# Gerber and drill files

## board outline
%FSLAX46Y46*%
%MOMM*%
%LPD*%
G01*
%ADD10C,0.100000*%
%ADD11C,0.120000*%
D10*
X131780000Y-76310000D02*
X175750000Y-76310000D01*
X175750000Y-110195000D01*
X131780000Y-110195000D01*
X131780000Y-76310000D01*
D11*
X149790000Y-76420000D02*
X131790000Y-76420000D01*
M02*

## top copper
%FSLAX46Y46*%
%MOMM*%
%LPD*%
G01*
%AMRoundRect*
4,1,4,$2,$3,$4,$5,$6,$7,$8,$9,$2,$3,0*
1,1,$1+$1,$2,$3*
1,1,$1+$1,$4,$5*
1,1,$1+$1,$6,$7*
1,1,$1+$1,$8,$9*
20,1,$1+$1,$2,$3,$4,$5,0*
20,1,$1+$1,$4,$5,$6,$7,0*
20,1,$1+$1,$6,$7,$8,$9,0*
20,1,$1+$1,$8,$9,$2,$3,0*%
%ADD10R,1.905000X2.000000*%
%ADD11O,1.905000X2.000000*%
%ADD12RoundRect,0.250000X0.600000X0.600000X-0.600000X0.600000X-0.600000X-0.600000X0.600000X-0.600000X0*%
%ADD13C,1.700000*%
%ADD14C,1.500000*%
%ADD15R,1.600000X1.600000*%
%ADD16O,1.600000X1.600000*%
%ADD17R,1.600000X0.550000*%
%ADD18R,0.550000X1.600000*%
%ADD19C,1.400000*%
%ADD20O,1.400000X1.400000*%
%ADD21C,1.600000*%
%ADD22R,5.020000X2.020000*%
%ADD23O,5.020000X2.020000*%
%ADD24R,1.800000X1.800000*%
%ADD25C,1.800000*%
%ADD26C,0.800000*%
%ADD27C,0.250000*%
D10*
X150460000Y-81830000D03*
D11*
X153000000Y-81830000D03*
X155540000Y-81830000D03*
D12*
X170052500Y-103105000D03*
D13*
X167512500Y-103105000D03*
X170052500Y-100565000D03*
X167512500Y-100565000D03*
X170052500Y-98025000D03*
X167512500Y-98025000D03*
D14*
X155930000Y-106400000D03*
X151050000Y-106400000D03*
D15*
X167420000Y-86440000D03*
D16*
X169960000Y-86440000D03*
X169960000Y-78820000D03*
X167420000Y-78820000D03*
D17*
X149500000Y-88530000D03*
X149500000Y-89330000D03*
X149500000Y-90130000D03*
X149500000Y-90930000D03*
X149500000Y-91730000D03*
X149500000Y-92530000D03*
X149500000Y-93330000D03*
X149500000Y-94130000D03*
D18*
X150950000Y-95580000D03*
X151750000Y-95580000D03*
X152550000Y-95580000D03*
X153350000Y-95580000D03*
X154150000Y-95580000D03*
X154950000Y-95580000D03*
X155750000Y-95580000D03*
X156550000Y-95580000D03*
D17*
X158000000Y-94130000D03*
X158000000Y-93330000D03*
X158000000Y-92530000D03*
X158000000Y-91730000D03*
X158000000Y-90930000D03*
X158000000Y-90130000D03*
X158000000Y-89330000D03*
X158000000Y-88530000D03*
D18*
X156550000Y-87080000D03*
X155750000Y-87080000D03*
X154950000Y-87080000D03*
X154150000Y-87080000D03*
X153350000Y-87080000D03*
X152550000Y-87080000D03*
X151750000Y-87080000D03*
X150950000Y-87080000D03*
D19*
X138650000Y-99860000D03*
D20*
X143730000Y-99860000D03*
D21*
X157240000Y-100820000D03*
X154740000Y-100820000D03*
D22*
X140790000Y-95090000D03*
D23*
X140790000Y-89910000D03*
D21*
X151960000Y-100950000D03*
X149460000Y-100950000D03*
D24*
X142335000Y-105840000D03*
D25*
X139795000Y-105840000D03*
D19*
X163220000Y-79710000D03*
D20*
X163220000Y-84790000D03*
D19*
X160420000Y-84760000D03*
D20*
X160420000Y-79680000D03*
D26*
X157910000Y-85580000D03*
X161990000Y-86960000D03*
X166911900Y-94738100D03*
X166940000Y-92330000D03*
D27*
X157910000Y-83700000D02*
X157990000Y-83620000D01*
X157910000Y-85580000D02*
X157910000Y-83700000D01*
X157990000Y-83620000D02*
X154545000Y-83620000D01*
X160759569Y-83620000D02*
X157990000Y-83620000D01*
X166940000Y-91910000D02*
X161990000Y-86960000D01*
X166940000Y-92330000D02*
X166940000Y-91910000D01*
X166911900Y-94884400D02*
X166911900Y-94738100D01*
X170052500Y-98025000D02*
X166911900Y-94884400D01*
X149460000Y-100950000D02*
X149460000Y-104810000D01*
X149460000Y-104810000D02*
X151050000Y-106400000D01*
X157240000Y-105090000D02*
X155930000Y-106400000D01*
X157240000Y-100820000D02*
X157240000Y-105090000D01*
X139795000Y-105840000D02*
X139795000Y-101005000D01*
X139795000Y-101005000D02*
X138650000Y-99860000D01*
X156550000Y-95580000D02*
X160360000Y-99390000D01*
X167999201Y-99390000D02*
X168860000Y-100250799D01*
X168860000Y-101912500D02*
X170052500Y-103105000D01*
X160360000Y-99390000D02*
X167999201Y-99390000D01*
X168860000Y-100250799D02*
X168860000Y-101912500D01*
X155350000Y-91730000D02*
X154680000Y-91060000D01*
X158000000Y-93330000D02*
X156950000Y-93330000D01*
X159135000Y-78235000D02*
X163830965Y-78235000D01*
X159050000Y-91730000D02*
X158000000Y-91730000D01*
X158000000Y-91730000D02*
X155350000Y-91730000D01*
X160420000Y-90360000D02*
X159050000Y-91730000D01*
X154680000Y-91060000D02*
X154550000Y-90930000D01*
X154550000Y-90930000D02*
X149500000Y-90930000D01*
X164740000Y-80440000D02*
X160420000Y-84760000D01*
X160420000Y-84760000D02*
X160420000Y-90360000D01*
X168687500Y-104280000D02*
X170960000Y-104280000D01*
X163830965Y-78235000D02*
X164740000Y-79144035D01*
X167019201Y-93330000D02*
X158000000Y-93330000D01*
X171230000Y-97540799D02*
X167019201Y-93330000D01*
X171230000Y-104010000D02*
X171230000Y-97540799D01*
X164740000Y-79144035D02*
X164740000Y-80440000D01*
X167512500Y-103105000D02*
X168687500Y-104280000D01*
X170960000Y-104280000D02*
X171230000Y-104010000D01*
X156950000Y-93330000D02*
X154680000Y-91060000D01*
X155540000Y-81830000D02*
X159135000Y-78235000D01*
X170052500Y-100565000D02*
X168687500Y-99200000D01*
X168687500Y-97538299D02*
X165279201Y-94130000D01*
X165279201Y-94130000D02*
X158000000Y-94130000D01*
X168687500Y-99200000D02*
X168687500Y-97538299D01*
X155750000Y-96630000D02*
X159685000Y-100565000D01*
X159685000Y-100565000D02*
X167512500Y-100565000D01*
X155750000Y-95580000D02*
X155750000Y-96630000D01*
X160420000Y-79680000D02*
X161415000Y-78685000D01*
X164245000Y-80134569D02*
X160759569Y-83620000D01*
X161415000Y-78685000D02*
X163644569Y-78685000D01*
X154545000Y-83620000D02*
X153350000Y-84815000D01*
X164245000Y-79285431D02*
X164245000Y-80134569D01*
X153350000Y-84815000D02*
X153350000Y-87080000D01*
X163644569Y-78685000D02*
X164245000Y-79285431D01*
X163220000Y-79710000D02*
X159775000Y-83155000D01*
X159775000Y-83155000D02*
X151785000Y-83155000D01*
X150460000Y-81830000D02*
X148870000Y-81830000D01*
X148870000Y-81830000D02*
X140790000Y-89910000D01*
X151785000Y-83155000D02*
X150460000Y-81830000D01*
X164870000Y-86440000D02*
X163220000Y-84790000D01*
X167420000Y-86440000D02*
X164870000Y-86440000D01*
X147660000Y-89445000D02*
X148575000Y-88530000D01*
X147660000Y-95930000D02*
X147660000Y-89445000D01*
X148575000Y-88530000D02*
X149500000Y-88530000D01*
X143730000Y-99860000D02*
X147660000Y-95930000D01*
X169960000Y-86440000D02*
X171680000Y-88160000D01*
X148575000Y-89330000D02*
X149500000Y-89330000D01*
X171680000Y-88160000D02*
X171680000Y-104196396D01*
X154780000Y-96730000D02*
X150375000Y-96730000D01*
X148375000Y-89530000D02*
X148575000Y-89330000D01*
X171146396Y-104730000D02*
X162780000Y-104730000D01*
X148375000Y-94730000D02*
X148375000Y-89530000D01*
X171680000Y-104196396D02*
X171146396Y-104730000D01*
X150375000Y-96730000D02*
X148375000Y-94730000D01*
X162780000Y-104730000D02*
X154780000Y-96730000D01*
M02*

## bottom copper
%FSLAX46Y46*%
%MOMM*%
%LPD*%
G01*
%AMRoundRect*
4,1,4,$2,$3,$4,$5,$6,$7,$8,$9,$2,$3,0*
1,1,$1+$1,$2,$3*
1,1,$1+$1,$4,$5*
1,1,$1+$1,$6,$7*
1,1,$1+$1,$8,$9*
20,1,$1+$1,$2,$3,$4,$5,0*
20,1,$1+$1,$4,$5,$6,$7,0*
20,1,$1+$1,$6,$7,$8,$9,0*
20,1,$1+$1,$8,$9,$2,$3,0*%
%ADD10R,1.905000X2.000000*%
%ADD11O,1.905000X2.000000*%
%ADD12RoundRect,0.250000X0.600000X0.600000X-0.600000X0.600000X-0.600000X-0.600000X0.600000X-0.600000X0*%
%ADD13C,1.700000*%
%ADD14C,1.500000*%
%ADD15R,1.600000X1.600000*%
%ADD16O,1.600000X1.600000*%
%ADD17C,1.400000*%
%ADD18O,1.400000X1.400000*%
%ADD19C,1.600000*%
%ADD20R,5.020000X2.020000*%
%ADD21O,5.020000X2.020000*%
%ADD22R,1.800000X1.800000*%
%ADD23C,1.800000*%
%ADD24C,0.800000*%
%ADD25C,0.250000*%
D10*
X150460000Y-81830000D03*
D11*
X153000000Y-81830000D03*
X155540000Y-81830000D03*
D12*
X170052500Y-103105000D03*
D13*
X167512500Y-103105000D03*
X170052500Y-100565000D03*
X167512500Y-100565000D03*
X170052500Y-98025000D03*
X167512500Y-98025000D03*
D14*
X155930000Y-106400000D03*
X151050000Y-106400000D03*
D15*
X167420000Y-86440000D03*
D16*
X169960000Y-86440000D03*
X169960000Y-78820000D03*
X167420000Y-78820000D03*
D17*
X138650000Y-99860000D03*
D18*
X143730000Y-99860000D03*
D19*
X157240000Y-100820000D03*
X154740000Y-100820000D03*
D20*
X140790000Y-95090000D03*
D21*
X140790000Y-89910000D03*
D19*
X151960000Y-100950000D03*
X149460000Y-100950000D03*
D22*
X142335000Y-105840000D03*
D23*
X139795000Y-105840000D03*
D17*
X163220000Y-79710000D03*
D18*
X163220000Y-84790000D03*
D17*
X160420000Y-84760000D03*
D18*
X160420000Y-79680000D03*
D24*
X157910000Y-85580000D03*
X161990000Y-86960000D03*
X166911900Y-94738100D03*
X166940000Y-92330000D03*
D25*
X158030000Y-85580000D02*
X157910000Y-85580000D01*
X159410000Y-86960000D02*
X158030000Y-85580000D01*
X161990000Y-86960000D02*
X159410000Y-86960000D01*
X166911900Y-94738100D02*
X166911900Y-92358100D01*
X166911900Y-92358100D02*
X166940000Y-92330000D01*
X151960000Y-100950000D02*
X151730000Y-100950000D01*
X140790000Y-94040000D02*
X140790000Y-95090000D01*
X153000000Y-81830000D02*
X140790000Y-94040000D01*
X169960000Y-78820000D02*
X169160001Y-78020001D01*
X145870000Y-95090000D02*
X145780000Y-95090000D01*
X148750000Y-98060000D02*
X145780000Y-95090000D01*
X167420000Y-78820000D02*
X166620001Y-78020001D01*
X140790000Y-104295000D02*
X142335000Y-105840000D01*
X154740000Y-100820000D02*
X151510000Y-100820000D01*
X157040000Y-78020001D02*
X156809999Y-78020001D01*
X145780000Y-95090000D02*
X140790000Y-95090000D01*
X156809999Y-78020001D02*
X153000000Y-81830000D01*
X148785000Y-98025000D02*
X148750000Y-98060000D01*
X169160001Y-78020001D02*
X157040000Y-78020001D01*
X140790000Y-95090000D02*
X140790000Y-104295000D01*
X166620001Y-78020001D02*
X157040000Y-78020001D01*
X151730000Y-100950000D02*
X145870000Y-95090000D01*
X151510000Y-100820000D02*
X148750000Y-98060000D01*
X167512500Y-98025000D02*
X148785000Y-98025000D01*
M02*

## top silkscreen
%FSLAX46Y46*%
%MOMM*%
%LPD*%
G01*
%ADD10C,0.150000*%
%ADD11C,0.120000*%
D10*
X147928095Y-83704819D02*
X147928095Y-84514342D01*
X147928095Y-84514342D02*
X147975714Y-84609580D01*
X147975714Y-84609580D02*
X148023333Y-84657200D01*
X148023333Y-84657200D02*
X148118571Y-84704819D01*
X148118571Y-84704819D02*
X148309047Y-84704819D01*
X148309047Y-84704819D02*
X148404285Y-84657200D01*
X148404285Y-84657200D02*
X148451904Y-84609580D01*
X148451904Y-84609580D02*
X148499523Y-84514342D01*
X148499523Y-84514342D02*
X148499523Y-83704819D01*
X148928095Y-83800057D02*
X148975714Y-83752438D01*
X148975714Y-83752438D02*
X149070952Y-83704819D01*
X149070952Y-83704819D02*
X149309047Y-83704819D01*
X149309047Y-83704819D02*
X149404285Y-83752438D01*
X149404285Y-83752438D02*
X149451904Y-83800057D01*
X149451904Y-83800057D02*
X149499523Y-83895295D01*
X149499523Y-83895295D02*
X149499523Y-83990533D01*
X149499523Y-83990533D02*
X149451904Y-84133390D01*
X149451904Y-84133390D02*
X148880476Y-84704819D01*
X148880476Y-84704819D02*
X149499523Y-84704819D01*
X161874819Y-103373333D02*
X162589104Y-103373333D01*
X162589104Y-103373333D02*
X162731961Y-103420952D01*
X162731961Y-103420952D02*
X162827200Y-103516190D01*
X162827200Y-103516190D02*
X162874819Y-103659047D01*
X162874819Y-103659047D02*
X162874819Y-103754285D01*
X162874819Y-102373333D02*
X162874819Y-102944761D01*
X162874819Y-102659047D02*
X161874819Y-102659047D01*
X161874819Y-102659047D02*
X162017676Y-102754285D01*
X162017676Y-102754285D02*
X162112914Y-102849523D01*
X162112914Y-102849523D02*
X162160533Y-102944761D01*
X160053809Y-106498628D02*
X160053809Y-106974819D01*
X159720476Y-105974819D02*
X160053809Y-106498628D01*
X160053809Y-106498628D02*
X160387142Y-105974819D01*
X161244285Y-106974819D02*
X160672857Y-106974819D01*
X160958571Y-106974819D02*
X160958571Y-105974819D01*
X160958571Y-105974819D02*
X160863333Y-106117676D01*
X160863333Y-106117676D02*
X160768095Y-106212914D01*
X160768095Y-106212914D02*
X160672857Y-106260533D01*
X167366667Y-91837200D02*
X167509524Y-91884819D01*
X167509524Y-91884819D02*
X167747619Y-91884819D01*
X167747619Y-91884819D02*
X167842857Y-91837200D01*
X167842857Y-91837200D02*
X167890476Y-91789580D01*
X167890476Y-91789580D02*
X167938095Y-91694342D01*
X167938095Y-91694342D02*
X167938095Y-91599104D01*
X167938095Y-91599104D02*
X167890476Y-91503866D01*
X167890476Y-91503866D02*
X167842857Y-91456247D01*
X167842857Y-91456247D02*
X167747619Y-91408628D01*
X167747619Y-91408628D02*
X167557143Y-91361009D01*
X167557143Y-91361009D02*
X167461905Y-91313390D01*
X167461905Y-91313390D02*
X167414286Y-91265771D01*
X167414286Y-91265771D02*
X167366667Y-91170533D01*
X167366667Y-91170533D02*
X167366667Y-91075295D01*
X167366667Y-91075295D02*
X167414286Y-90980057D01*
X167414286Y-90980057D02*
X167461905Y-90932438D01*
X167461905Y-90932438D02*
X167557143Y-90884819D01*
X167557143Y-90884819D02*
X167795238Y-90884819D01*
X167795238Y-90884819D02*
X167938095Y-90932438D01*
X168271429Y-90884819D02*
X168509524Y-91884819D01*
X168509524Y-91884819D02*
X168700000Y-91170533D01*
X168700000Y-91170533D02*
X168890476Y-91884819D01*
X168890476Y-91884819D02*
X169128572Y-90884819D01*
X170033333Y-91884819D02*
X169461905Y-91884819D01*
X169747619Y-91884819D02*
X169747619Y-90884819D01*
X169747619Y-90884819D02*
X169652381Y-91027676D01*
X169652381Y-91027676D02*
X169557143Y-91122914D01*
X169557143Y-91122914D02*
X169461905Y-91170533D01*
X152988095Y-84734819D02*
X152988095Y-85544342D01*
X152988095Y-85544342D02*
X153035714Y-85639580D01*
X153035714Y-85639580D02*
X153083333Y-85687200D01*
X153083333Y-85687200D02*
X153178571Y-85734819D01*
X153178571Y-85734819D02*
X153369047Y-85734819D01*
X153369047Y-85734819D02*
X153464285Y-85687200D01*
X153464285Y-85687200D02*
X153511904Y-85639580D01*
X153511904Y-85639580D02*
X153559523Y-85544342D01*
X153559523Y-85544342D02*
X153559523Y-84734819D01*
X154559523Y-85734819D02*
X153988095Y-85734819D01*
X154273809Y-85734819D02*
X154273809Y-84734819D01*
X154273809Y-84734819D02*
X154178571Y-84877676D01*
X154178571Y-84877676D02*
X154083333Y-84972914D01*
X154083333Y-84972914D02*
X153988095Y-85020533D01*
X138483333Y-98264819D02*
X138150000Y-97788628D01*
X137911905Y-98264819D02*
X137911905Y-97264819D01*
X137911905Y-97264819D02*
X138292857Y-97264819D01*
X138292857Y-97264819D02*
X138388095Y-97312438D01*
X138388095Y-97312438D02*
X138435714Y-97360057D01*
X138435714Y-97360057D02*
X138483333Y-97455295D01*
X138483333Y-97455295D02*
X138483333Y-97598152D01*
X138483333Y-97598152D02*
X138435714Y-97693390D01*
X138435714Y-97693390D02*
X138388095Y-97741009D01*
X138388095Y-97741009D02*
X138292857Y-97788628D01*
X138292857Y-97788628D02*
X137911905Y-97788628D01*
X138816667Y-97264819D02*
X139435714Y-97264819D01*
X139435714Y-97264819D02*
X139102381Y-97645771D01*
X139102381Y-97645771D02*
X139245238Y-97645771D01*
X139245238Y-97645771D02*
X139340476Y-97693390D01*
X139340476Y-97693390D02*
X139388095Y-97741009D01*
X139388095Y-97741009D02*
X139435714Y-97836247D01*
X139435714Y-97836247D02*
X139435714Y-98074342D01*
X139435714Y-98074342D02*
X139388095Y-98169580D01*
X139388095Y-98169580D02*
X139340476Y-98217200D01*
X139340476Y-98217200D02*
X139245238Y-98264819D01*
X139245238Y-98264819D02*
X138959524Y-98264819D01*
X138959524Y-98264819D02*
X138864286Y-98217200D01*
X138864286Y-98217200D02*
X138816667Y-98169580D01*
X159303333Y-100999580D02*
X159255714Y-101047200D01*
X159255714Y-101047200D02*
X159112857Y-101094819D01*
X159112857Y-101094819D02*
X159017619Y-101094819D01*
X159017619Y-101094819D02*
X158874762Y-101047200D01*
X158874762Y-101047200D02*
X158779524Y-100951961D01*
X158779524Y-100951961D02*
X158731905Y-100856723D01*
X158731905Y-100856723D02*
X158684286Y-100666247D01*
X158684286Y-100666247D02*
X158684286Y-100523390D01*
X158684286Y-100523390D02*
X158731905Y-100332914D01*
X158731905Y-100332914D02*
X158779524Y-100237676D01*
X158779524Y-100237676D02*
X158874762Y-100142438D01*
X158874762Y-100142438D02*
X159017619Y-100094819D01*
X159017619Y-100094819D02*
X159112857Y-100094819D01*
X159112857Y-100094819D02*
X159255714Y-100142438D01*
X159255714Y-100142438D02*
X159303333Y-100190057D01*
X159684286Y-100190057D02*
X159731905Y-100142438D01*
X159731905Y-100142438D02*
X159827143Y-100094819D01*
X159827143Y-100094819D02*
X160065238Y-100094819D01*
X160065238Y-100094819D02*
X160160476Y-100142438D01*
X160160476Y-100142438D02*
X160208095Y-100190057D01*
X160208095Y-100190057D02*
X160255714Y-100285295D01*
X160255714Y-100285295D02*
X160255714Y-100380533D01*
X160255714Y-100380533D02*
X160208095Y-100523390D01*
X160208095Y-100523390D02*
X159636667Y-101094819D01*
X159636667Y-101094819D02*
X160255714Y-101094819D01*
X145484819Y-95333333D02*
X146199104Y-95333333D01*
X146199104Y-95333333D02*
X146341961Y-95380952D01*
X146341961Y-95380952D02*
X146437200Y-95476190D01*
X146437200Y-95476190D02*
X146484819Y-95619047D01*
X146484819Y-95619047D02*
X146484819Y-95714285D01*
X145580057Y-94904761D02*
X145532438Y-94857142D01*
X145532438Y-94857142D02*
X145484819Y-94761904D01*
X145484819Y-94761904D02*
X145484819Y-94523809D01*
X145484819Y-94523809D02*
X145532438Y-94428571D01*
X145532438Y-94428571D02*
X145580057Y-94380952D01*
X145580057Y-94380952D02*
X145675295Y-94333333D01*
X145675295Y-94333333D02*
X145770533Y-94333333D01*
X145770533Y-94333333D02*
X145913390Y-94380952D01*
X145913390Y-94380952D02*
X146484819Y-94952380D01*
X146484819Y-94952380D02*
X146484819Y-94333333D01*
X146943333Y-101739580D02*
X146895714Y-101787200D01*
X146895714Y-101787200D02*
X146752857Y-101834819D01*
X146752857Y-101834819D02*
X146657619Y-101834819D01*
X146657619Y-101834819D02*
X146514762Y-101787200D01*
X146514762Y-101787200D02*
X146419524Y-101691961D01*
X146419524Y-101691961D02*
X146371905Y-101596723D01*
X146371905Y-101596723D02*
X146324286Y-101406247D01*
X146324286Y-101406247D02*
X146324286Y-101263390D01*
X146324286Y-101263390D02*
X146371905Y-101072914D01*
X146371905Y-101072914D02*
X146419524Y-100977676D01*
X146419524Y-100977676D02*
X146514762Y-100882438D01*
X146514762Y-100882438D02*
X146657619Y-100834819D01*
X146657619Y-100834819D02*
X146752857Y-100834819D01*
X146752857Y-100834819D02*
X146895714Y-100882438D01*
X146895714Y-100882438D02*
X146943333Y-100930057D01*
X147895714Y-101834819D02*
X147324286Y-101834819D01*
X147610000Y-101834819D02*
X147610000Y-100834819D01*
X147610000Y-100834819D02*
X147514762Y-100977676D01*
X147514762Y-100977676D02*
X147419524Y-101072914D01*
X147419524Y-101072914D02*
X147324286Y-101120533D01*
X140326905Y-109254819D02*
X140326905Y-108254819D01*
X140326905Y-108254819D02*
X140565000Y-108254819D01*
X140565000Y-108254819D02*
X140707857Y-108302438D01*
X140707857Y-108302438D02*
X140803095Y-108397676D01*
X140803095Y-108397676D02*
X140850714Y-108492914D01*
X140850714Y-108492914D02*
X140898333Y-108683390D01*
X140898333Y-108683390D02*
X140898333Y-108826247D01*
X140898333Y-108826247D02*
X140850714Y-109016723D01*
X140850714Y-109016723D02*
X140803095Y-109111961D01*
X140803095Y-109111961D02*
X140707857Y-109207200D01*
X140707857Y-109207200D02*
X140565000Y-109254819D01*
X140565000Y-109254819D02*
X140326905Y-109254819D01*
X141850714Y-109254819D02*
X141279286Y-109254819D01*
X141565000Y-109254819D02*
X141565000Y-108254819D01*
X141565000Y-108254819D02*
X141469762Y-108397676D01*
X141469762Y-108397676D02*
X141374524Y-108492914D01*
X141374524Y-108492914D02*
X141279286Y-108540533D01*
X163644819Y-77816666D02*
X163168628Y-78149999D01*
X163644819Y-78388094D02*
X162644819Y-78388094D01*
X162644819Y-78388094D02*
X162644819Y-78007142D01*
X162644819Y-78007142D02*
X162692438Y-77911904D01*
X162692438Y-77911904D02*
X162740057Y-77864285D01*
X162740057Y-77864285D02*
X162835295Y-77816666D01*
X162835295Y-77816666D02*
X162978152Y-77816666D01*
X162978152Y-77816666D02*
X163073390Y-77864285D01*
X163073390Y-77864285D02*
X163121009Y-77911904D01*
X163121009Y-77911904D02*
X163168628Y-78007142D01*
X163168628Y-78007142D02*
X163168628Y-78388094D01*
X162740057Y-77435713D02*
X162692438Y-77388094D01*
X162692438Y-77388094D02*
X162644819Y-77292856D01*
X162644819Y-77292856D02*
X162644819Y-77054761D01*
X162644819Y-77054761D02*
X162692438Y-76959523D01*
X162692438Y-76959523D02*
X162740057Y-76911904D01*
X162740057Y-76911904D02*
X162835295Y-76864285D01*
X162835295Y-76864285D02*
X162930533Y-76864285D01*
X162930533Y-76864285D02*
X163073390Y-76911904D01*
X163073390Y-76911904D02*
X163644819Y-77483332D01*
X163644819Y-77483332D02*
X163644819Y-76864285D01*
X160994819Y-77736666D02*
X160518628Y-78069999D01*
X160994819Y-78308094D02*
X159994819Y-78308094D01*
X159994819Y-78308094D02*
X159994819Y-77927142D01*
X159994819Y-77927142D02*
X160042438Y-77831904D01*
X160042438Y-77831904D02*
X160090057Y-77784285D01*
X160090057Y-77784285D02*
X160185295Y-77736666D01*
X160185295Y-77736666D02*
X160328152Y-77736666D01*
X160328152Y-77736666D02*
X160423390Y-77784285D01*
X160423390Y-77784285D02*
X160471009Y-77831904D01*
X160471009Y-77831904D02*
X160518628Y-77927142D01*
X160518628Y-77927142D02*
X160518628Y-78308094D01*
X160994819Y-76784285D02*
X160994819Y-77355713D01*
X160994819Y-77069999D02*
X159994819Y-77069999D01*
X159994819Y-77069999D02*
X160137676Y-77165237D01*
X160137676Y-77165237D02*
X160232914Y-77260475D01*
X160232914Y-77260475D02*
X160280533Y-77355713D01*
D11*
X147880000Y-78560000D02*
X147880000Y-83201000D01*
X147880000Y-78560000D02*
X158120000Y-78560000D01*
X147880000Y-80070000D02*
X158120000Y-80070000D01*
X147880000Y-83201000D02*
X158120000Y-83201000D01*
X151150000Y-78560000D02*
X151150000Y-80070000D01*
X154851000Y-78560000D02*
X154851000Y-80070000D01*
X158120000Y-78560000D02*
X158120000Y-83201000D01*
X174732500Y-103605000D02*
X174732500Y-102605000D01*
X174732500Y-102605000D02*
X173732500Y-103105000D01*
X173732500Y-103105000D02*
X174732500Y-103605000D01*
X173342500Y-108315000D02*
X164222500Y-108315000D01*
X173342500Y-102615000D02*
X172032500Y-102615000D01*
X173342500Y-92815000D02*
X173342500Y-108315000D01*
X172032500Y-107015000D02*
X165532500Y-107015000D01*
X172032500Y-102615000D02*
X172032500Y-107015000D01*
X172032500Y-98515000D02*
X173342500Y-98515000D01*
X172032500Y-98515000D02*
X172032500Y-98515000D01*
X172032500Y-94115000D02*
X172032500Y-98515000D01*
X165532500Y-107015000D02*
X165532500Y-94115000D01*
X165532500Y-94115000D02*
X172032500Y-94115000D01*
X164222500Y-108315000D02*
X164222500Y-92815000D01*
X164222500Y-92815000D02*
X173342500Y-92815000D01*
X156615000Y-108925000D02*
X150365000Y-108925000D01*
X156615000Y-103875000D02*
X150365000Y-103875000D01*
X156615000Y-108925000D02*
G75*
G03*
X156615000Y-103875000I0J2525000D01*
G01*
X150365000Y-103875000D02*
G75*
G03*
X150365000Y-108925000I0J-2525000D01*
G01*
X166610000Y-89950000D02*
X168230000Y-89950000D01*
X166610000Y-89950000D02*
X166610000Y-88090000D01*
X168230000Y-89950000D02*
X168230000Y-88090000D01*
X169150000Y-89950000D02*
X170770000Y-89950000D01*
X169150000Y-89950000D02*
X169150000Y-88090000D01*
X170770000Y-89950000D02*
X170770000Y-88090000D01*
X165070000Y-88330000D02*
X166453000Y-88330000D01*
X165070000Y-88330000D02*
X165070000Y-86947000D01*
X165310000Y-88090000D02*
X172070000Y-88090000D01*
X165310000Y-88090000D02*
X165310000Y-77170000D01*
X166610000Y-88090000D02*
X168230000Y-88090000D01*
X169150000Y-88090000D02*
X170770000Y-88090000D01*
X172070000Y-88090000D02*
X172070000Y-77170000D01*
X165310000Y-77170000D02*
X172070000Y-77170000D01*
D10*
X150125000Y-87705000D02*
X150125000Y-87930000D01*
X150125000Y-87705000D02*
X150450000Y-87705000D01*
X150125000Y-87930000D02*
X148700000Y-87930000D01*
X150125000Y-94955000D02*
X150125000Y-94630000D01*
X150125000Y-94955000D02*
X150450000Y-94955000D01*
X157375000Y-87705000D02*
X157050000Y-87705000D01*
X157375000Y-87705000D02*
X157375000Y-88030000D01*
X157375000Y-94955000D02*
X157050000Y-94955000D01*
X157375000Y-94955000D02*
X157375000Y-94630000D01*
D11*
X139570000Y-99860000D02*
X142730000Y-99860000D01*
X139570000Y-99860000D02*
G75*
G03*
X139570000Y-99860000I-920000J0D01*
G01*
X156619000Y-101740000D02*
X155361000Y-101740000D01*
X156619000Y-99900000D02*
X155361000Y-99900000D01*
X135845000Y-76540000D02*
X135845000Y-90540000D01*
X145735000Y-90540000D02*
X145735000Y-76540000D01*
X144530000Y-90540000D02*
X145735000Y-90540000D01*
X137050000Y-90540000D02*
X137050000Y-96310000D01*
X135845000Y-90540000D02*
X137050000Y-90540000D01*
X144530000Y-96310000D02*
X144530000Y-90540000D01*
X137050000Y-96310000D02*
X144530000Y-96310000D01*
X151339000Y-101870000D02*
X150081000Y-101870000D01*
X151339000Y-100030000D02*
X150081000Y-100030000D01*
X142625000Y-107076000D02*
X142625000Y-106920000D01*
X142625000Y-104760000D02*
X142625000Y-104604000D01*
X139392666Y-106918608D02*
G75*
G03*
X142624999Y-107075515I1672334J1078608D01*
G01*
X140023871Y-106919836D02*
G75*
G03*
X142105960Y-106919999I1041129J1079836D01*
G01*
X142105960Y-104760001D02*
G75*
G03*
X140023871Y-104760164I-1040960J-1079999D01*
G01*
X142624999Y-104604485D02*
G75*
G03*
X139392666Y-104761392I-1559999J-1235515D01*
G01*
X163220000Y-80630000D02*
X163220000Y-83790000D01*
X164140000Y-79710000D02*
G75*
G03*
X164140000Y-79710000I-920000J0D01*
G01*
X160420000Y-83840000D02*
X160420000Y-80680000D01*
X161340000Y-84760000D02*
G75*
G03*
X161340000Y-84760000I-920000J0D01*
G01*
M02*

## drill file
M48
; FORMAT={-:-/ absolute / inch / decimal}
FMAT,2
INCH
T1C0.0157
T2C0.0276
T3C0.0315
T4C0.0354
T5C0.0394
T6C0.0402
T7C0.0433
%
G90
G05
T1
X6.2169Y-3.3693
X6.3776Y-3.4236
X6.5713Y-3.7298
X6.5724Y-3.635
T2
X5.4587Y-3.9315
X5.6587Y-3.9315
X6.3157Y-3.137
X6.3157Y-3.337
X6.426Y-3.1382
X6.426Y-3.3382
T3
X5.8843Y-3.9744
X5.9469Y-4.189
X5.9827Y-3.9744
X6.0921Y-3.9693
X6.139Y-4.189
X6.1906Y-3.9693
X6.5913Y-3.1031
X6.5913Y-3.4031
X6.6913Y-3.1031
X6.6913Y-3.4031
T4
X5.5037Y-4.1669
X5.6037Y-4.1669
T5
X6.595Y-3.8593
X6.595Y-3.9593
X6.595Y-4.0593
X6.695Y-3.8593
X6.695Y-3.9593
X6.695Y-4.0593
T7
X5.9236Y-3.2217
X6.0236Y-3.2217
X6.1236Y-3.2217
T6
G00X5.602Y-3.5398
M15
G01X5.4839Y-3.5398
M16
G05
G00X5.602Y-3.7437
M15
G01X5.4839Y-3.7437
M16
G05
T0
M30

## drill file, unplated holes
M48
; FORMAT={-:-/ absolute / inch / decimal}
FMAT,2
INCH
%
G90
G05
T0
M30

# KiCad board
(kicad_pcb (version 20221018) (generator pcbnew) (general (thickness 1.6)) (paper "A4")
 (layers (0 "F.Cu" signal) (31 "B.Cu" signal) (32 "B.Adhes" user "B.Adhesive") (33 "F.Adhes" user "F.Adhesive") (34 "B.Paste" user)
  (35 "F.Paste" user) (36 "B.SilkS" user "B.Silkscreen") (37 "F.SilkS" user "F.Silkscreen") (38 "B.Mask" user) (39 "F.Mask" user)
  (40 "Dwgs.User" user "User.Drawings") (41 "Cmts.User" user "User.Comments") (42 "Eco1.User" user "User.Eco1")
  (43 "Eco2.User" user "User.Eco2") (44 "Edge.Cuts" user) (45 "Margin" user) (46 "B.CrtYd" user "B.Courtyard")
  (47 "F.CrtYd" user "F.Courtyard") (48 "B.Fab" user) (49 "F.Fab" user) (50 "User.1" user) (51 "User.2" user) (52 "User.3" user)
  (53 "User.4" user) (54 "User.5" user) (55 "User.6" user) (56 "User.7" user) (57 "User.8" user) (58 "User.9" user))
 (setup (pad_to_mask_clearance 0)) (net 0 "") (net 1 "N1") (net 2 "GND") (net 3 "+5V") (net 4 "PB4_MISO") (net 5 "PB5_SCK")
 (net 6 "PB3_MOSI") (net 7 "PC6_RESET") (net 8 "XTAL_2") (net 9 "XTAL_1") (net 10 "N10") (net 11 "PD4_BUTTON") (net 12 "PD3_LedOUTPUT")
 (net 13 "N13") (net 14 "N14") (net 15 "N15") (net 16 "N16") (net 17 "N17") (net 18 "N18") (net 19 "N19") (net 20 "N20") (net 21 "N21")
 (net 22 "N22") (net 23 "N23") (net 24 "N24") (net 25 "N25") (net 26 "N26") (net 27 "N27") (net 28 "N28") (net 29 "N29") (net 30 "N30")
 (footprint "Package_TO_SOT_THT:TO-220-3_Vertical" (layer "F.Cu") (at 150.46 81.83)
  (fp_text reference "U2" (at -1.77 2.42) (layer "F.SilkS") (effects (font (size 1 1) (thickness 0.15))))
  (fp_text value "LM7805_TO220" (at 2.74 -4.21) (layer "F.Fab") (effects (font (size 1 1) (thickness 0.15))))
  (fp_line (start -2.58 -3.27) (end -2.58 1.371) (stroke (width 0.12) (type solid)) (layer "F.SilkS"))
  (fp_line (start -2.58 -3.27) (end 7.66 -3.27) (stroke (width 0.12) (type solid)) (layer "F.SilkS"))
  (fp_line (start -2.58 -1.76) (end 7.66 -1.76) (stroke (width 0.12) (type solid)) (layer "F.SilkS"))
  (fp_line (start -2.58 1.371) (end 7.66 1.371) (stroke (width 0.12) (type solid)) (layer "F.SilkS"))
  (fp_line (start 0.69 -3.27) (end 0.69 -1.76) (stroke (width 0.12) (type solid)) (layer "F.SilkS"))
  (fp_line (start 4.391 -3.27) (end 4.391 -1.76) (stroke (width 0.12) (type solid)) (layer "F.SilkS"))
  (fp_line (start 7.66 -3.27) (end 7.66 1.371) (stroke (width 0.12) (type solid)) (layer "F.SilkS"))
  (pad "1" thru_hole rect (at 0 0) (size 1.905 2) (drill 1.1) (layers "*.Cu" "*.Mask") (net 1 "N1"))
  (pad "2" thru_hole oval (at 2.54 0) (size 1.905 2) (drill 1.1) (layers "*.Cu" "*.Mask") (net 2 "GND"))
  (pad "3" thru_hole oval (at 5.08 0) (size 1.905 2) (drill 1.1) (layers "*.Cu" "*.Mask") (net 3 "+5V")))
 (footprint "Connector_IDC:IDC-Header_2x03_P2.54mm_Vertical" (layer "F.Cu") (at 170.0525 103.105 180)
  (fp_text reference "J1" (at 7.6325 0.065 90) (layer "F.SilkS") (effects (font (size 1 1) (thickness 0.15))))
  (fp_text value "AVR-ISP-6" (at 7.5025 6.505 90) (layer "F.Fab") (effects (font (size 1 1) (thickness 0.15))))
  (fp_line (start -4.68 -0.5) (end -4.68 0.5) (stroke (width 0.12) (type solid)) (layer "F.SilkS"))
  (fp_line (start -4.68 0.5) (end -3.68 0) (stroke (width 0.12) (type solid)) (layer "F.SilkS"))
  (fp_line (start -3.68 0) (end -4.68 -0.5) (stroke (width 0.12) (type solid)) (layer "F.SilkS"))
  (fp_line (start -3.29 -5.21) (end 5.83 -5.21) (stroke (width 0.12) (type solid)) (layer "F.SilkS"))
  (fp_line (start -3.29 0.49) (end -1.98 0.49) (stroke (width 0.12) (type solid)) (layer "F.SilkS"))
  (fp_line (start -3.29 10.29) (end -3.29 -5.21) (stroke (width 0.12) (type solid)) (layer "F.SilkS"))
  (fp_line (start -1.98 -3.91) (end 4.52 -3.91) (stroke (width 0.12) (type solid)) (layer "F.SilkS"))
  (fp_line (start -1.98 0.49) (end -1.98 -3.91) (stroke (width 0.12) (type solid)) (layer "F.SilkS"))
  (fp_line (start -1.98 4.59) (end -3.29 4.59) (stroke (width 0.12) (type solid)) (layer "F.SilkS"))
  (fp_line (start -1.98 4.59) (end -1.98 4.59) (stroke (width 0.12) (type solid)) (layer "F.SilkS"))
  (fp_line (start -1.98 8.99) (end -1.98 4.59) (stroke (width 0.12) (type solid)) (layer "F.SilkS"))
  (fp_line (start 4.52 -3.91) (end 4.52 8.99) (stroke (width 0.12) (type solid)) (layer "F.SilkS"))
  (fp_line (start 4.52 8.99) (end -1.98 8.99) (stroke (width 0.12) (type solid)) (layer "F.SilkS"))
  (fp_line (start 5.83 -5.21) (end 5.83 10.29) (stroke (width 0.12) (type solid)) (layer "F.SilkS"))
  (fp_line (start 5.83 10.29) (end -3.29 10.29) (stroke (width 0.12) (type solid)) (layer "F.SilkS"))
  (pad "1" thru_hole roundrect (at 0 0 180) (size 1.7 1.7) (drill 1) (layers "*.Cu" "*.Mask") (roundrect_rratio 0.1470588235)
   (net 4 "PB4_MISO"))
  (pad "2" thru_hole circle (at 2.54 0 180) (size 1.7 1.7) (drill 1) (layers "*.Cu" "*.Mask") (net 3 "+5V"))
  (pad "3" thru_hole circle (at 0 2.54 180) (size 1.7 1.7) (drill 1) (layers "*.Cu" "*.Mask") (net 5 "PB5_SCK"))
  (pad "4" thru_hole circle (at 2.54 2.54 180) (size 1.7 1.7) (drill 1) (layers "*.Cu" "*.Mask") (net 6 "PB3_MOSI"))
  (pad "5" thru_hole circle (at 0 5.08 180) (size 1.7 1.7) (drill 1) (layers "*.Cu" "*.Mask") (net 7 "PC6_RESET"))
  (pad "6" thru_hole circle (at 2.54 5.08 180) (size 1.7 1.7) (drill 1) (layers "*.Cu" "*.Mask") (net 2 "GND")))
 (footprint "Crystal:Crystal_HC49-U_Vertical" (layer "F.Cu") (at 155.93 106.4 180)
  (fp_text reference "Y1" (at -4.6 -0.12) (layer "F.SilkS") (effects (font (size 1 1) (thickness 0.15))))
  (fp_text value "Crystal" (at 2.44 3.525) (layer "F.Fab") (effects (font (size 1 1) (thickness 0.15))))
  (fp_line (start -0.685 -2.525) (end 5.565 -2.525) (stroke (width 0.12) (type solid)) (layer "F.SilkS"))
  (fp_line (start -0.685 2.525) (end 5.565 2.525) (stroke (width 0.12) (type solid)) (layer "F.SilkS"))
  (fp_arc (start -0.685 2.525) (mid -3.21 0) (end -0.685 -2.525) (stroke (width 0.12) (type solid)) (layer "F.SilkS"))
  (fp_arc (start 5.565 -2.525) (mid 8.09 0) (end 5.565 2.525) (stroke (width 0.12) (type solid)) (layer "F.SilkS"))
  (pad "1" thru_hole circle (at 0 0 180) (size 1.5 1.5) (drill 0.8) (layers "*.Cu" "*.Mask") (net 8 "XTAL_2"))
  (pad "2" thru_hole circle (at 4.88 0 180) (size 1.5 1.5) (drill 0.8) (layers "*.Cu" "*.Mask") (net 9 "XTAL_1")))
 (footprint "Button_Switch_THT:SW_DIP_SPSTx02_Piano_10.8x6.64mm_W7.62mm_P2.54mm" (layer "F.Cu") (at 167.42 86.44 90)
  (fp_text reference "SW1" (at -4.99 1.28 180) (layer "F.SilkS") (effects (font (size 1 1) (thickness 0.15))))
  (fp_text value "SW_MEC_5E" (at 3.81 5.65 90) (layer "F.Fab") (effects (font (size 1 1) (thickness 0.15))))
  (fp_line (start -3.51 -0.81) (end -3.51 0.81) (stroke (width 0.12) (type solid)) (layer "F.SilkS"))
  (fp_line (start -3.51 -0.81) (end -1.65 -0.81) (stroke (width 0.12) (type solid)) (layer "F.SilkS"))
  (fp_line (start -3.51 0.81) (end -1.65 0.81) (stroke (width 0.12) (type solid)) (layer "F.SilkS"))
  (fp_line (start -3.51 1.73) (end -3.51 3.35) (stroke (width 0.12) (type solid)) (layer "F.SilkS"))
  (fp_line (start -3.51 1.73) (end -1.65 1.73) (stroke (width 0.12) (type solid)) (layer "F.SilkS"))
  (fp_line (start -3.51 3.35) (end -1.65 3.35) (stroke (width 0.12) (type solid)) (layer "F.SilkS"))
  (fp_line (start -1.89 -2.35) (end -1.89 -0.967) (stroke (width 0.12) (type solid)) (layer "F.SilkS"))
  (fp_line (start -1.89 -2.35) (end -0.507 -2.35) (stroke (width 0.12) (type solid)) (layer "F.SilkS"))
  (fp_line (start -1.65 -2.11) (end -1.65 4.65) (stroke (width 0.12) (type solid)) (layer "F.SilkS"))
  (fp_line (start -1.65 -2.11) (end 9.27 -2.11) (stroke (width 0.12) (type solid)) (layer "F.SilkS"))
  (fp_line (start -1.65 -0.81) (end -1.65 0.81) (stroke (width 0.12) (type solid)) (layer "F.SilkS"))
  (fp_line (start -1.65 1.73) (end -1.65 3.35) (stroke (width 0.12) (type solid)) (layer "F.SilkS"))
  (fp_line (start -1.65 4.65) (end 9.27 4.65) (stroke (width 0.12) (type solid)) (layer "F.SilkS"))
  (fp_line (start 9.27 -2.11) (end 9.27 4.65) (stroke (width 0.12) (type solid)) (layer "F.SilkS"))
  (pad "1" thru_hole rect (at 0 0 90) (size 1.6 1.6) (drill 0.8) (layers "*.Cu" "*.Mask") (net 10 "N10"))
  (pad "2" thru_hole oval (at 0 2.54 90) (size 1.6 1.6) (drill 0.8) (layers "*.Cu" "*.Mask") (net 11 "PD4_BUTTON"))
  (pad "3" thru_hole oval (at 7.62 2.54 90) (size 1.6 1.6) (drill 0.8) (layers "*.Cu" "*.Mask") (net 2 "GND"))
  (pad "4" thru_hole oval (at 7.62 0 90) (size 1.6 1.6) (drill 0.8) (layers "*.Cu" "*.Mask") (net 2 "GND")))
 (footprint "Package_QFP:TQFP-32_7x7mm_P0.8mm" (layer "F.Cu") (at 153.75 91.33)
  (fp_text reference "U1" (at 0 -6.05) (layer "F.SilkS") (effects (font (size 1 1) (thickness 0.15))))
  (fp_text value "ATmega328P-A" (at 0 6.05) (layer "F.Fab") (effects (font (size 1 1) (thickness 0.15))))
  (fp_line (start -3.625 -3.625) (end -3.625 -3.4) (stroke (width 0.15) (type solid)) (layer "F.SilkS"))
  (fp_line (start -3.625 -3.625) (end -3.3 -3.625) (stroke (width 0.15) (type solid)) (layer "F.SilkS"))
  (fp_line (start -3.625 -3.4) (end -5.05 -3.4) (stroke (width 0.15) (type solid)) (layer "F.SilkS"))
  (fp_line (start -3.625 3.625) (end -3.625 3.3) (stroke (width 0.15) (type solid)) (layer "F.SilkS"))
  (fp_line (start -3.625 3.625) (end -3.3 3.625) (stroke (width 0.15) (type solid)) (layer "F.SilkS"))
  (fp_line (start 3.625 -3.625) (end 3.3 -3.625) (stroke (width 0.15) (type solid)) (layer "F.SilkS"))
  (fp_line (start 3.625 -3.625) (end 3.625 -3.3) (stroke (width 0.15) (type solid)) (layer "F.SilkS"))
  (fp_line (start 3.625 3.625) (end 3.3 3.625) (stroke (width 0.15) (type solid)) (layer "F.SilkS"))
  (fp_line (start 3.625 3.625) (end 3.625 3.3) (stroke (width 0.15) (type solid)) (layer "F.SilkS"))
  (pad "1" smd rect (at -4.25 -2.8) (size 1.6 0.55) (layers "F.Cu" "F.Paste" "F.Mask") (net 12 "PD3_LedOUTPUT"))
  (pad "2" smd rect (at -4.25 -2) (size 1.6 0.55) (layers "F.Cu" "F.Paste" "F.Mask") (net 11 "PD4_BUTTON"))
  (pad "3" smd rect (at -4.25 -1.2) (size 1.6 0.55) (layers "F.Cu" "F.Paste" "F.Mask") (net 2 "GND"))
  (pad "4" smd rect (at -4.25 -0.4) (size 1.6 0.55) (layers "F.Cu" "F.Paste" "F.Mask") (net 3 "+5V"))
  (pad "5" smd rect (at -4.25 0.4) (size 1.6 0.55) (layers "F.Cu" "F.Paste" "F.Mask") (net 2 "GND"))
  (pad "6" smd rect (at -4.25 1.2) (size 1.6 0.55) (layers "F.Cu" "F.Paste" "F.Mask") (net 3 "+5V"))
  (pad "7" smd rect (at -4.25 2) (size 1.6 0.55) (layers "F.Cu" "F.Paste" "F.Mask") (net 9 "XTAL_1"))
  (pad "8" smd rect (at -4.25 2.8) (size 1.6 0.55) (layers "F.Cu" "F.Paste" "F.Mask") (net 8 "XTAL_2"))
  (pad "9" smd rect (at -2.8 4.25 90) (size 1.6 0.55) (layers "F.Cu" "F.Paste" "F.Mask") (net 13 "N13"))
  (pad "10" smd rect (at -2 4.25 90) (size 1.6 0.55) (layers "F.Cu" "F.Paste" "F.Mask") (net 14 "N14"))
  (pad "11" smd rect (at -1.2 4.25 90) (size 1.6 0.55) (layers "F.Cu" "F.Paste" "F.Mask") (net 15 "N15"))
  (pad "12" smd rect (at -0.4 4.25 90) (size 1.6 0.55) (layers "F.Cu" "F.Paste" "F.Mask") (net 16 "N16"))
  (pad "13" smd rect (at 0.4 4.25 90) (size 1.6 0.55) (layers "F.Cu" "F.Paste" "F.Mask") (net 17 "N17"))
  (pad "14" smd rect (at 1.2 4.25 90) (size 1.6 0.55) (layers "F.Cu" "F.Paste" "F.Mask") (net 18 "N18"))
  (pad "15" smd rect (at 2 4.25 90) (size 1.6 0.55) (layers "F.Cu" "F.Paste" "F.Mask") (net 6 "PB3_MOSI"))
  (pad "16" smd rect (at 2.8 4.25 90) (size 1.6 0.55) (layers "F.Cu" "F.Paste" "F.Mask") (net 4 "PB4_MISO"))
  (pad "17" smd rect (at 4.25 2.8) (size 1.6 0.55) (layers "F.Cu" "F.Paste" "F.Mask") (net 5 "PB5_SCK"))
  (pad "18" smd rect (at 4.25 2) (size 1.6 0.55) (layers "F.Cu" "F.Paste" "F.Mask") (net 3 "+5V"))
  (pad "19" smd rect (at 4.25 1.2) (size 1.6 0.55) (layers "F.Cu" "F.Paste" "F.Mask") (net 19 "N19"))
  (pad "20" smd rect (at 4.25 0.4) (size 1.6 0.55) (layers "F.Cu" "F.Paste" "F.Mask") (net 3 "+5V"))
  (pad "21" smd rect (at 4.25 -0.4) (size 1.6 0.55) (layers "F.Cu" "F.Paste" "F.Mask") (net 2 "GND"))
  (pad "22" smd rect (at 4.25 -1.2) (size 1.6 0.55) (layers "F.Cu" "F.Paste" "F.Mask") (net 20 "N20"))
  (pad "23" smd rect (at 4.25 -2) (size 1.6 0.55) (layers "F.Cu" "F.Paste" "F.Mask") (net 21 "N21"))
  (pad "24" smd rect (at 4.25 -2.8) (size 1.6 0.55) (layers "F.Cu" "F.Paste" "F.Mask") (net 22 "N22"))
  (pad "25" smd rect (at 2.8 -4.25 90) (size 1.6 0.55) (layers "F.Cu" "F.Paste" "F.Mask") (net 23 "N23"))
  (pad "26" smd rect (at 2 -4.25 90) (size 1.6 0.55) (layers "F.Cu" "F.Paste" "F.Mask") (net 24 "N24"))
  (pad "27" smd rect (at 1.2 -4.25 90) (size 1.6 0.55) (layers "F.Cu" "F.Paste" "F.Mask") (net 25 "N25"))
  (pad "28" smd rect (at 0.4 -4.25 90) (size 1.6 0.55) (layers "F.Cu" "F.Paste" "F.Mask") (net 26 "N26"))
  (pad "29" smd rect (at -0.4 -4.25 90) (size 1.6 0.55) (layers "F.Cu" "F.Paste" "F.Mask") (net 7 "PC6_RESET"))
  (pad "30" smd rect (at -1.2 -4.25 90) (size 1.6 0.55) (layers "F.Cu" "F.Paste" "F.Mask") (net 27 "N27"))
  (pad "31" smd rect (at -2 -4.25 90) (size 1.6 0.55) (layers "F.Cu" "F.Paste" "F.Mask") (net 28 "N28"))
  (pad "32" smd rect (at -2.8 -4.25 90) (size 1.6 0.55) (layers "F.Cu" "F.Paste" "F.Mask") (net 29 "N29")))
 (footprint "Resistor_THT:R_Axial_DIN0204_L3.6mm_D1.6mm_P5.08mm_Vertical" (layer "F.Cu") (at 138.65 99.86)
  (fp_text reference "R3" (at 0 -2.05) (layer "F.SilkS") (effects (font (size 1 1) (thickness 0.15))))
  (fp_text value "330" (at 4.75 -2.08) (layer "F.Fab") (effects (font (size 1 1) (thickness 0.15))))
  (fp_line (start 0.92 0) (end 4.08 0) (stroke (width 0.12) (type solid)) (layer "F.SilkS"))
  (fp_circle (center 0 0) (end 0.92 0) (stroke (width 0.12) (type solid)) (fill none) (layer "F.SilkS"))
  (pad "1" thru_hole circle (at 0 0) (size 1.4 1.4) (drill 0.7) (layers "*.Cu" "*.Mask") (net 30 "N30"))
  (pad "2" thru_hole oval (at 5.08 0) (size 1.4 1.4) (drill 0.7) (layers "*.Cu" "*.Mask") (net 12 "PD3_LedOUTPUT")))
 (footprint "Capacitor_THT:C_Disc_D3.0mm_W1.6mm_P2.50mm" (layer "F.Cu") (at 157.24 100.82 180)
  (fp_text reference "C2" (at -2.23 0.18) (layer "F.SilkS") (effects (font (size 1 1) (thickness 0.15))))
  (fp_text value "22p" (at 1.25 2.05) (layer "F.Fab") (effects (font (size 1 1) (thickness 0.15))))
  (fp_line (start 0.621 -0.92) (end 1.879 -0.92) (stroke (width 0.12) (type solid)) (layer "F.SilkS"))
  (fp_line (start 0.621 0.92) (end 1.879 0.92) (stroke (width 0.12) (type solid)) (layer "F.SilkS"))
  (pad "1" thru_hole circle (at 0 0 180) (size 1.6 1.6) (drill 0.8) (layers "*.Cu" "*.Mask") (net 8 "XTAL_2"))
  (pad "2" thru_hole circle (at 2.5 0 180) (size 1.6 1.6) (drill 0.8) (layers "*.Cu" "*.Mask") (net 2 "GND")))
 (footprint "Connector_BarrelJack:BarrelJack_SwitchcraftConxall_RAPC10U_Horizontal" (layer "F.Cu") (at 140.79 95.09 -90)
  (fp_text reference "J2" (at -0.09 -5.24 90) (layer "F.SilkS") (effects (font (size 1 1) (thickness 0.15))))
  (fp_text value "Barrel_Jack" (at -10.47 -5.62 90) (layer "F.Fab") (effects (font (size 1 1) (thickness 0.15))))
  (fp_line (start -18.55 4.945) (end -4.55 4.945) (stroke (width 0.12) (type solid)) (layer "F.SilkS"))
  (fp_line (start -4.55 -4.945) (end -18.55 -4.945) (stroke (width 0.12) (type solid)) (layer "F.SilkS"))
  (fp_line (start -4.55 -3.74) (end -4.55 -4.945) (stroke (width 0.12) (type solid)) (layer "F.SilkS"))
  (fp_line (start -4.55 3.74) (end 1.22 3.74) (stroke (width 0.12) (type solid)) (layer "F.SilkS"))
  (fp_line (start -4.55 4.945) (end -4.55 3.74) (stroke (width 0.12) (type solid)) (layer "F.SilkS"))
  (fp_line (start 1.22 -3.74) (end -4.55 -3.74) (stroke (width 0.12) (type solid)) (layer "F.SilkS"))
  (fp_line (start 1.22 3.74) (end 1.22 -3.74) (stroke (width 0.12) (type solid)) (layer "F.SilkS"))
  (fp_line (start -18.67 -9) (end -18.67 9) (stroke (width 0.12) (type solid)) (layer "Edge.Cuts"))
  (pad "1" thru_hole rect (at 0 0 270) (size 2.02 5.02) (drill oval 1.02 4.02) (layers "*.Cu" "*.Mask") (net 2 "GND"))
  (pad "2" thru_hole oval (at -5.18 0 270) (size 2.02 5.02) (drill oval 1.02 4.02) (layers "*.Cu" "*.Mask") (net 1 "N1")))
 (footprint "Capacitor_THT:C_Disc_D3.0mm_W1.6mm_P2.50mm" (layer "F.Cu") (at 151.96 100.95 180)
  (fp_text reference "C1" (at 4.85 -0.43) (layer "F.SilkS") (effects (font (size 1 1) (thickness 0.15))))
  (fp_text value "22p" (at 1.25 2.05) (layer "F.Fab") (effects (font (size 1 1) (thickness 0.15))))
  (fp_line (start 0.621 -0.92) (end 1.879 -0.92) (stroke (width 0.12) (type solid)) (layer "F.SilkS"))
  (fp_line (start 0.621 0.92) (end 1.879 0.92) (stroke (width 0.12) (type solid)) (layer "F.SilkS"))
  (pad "1" thru_hole circle (at 0 0 180) (size 1.6 1.6) (drill 0.8) (layers "*.Cu" "*.Mask") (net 2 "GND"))
  (pad "2" thru_hole circle (at 2.5 0 180) (size 1.6 1.6) (drill 0.8) (layers "*.Cu" "*.Mask") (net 9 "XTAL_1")))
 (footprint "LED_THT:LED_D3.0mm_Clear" (layer "F.Cu") (at 142.335 105.84 180)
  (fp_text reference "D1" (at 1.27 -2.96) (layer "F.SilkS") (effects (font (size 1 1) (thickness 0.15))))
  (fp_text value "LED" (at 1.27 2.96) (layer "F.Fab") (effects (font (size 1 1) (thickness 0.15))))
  (fp_line (start -0.29 -1.236) (end -0.29 -1.08) (stroke (width 0.12) (type solid)) (layer "F.SilkS"))
  (fp_line (start -0.29 1.08) (end -0.29 1.236) (stroke (width 0.12) (type solid)) (layer "F.SilkS"))
  (fp_arc (start -0.29 -1.235516) (mid 1.366487 -1.987659) (end 2.942335 -1.078608) (stroke (width 0.12) (type solid)) (layer "F.SilkS"))
  (fp_arc (start 0.229039 -1.08) (mid 1.270117 -1.5) (end 2.31113 -1.079837) (stroke (width 0.12) (type solid)) (layer "F.SilkS"))
  (fp_arc (start 2.31113 1.079837) (mid 1.270117 1.5) (end 0.229039 1.08) (stroke (width 0.12) (type solid)) (layer "F.SilkS"))
  (fp_arc (start 2.942335 1.078608) (mid 1.366487 1.987659) (end -0.29 1.235516) (stroke (width 0.12) (type solid)) (layer "F.SilkS"))
  (pad "1" thru_hole rect (at 0 0 180) (size 1.8 1.8) (drill 0.9) (layers "*.Cu" "*.Mask") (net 2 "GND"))
  (pad "2" thru_hole circle (at 2.54 0 180) (size 1.8 1.8) (drill 0.9) (layers "*.Cu" "*.Mask") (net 30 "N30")))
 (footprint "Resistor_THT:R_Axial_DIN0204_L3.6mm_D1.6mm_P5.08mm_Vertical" (layer "F.Cu") (at 163.22 79.71 -90)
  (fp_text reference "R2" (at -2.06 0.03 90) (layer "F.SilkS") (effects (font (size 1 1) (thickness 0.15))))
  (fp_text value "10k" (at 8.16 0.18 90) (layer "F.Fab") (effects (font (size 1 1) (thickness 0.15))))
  (fp_line (start 0.92 0) (end 4.08 0) (stroke (width 0.12) (type solid)) (layer "F.SilkS"))
  (fp_circle (center 0 0) (end 0.92 0) (stroke (width 0.12) (type solid)) (fill none) (layer "F.SilkS"))
  (pad "1" thru_hole circle (at 0 0 270) (size 1.4 1.4) (drill 0.7) (layers "*.Cu" "*.Mask") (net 1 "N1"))
  (pad "2" thru_hole oval (at 5.08 0 270) (size 1.4 1.4) (drill 0.7) (layers "*.Cu" "*.Mask") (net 10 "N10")))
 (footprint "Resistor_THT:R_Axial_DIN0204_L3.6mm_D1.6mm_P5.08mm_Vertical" (layer "F.Cu") (at 160.42 84.76 90)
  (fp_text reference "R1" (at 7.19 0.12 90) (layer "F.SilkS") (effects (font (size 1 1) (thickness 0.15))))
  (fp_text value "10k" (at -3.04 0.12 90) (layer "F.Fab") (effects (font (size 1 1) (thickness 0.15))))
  (fp_line (start 0.92 0) (end 4.08 0) (stroke (width 0.12) (type solid)) (layer "F.SilkS"))
  (fp_circle (center 0 0) (end 0.92 0) (stroke (width 0.12) (type solid)) (fill none) (layer "F.SilkS"))
  (pad "1" thru_hole circle (at 0 0 90) (size 1.4 1.4) (drill 0.7) (layers "*.Cu" "*.Mask") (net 3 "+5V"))
  (pad "2" thru_hole oval (at 5.08 0 90) (size 1.4 1.4) (drill 0.7) (layers "*.Cu" "*.Mask") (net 7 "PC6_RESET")))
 (gr_rect (start 131.78 76.31) (end 175.75 110.195) (stroke (width 0.1) (type default)) (fill none) (layer "Edge.Cuts"))
 (segment (start 151.96 100.95) (end 151.73 100.95) (width 0.25) (layer "B.Cu") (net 2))
 (segment (start 140.79 94.04) (end 140.79 95.09) (width 0.25) (layer "B.Cu") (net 2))
 (segment (start 153 81.83) (end 140.79 94.04) (width 0.25) (layer "B.Cu") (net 2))
 (segment (start 169.96 78.82) (end 169.160001 78.020001) (width 0.25) (layer "B.Cu") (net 2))
 (segment (start 145.87 95.09) (end 145.78 95.09) (width 0.25) (layer "B.Cu") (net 2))
 (segment (start 148.75 98.06) (end 145.78 95.09) (width 0.25) (layer "B.Cu") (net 2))
 (segment (start 167.42 78.82) (end 166.620001 78.020001) (width 0.25) (layer "B.Cu") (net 2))
 (segment (start 140.79 104.295) (end 142.335 105.84) (width 0.25) (layer "B.Cu") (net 2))
 (segment (start 154.74 100.82) (end 151.51 100.82) (width 0.25) (layer "B.Cu") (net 2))
 (segment (start 157.04 78.020001) (end 156.809999 78.020001) (width 0.25) (layer "B.Cu") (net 2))
 (segment (start 145.78 95.09) (end 140.79 95.09) (width 0.25) (layer "B.Cu") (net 2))
 (segment (start 156.809999 78.020001) (end 153 81.83) (width 0.25) (layer "B.Cu") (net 2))
 (segment (start 148.785 98.025) (end 148.75 98.06) (width 0.25) (layer "B.Cu") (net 2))
 (segment (start 169.160001 78.020001) (end 157.04 78.020001) (width 0.25) (layer "B.Cu") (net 2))
 (segment (start 140.79 95.09) (end 140.79 104.295) (width 0.25) (layer "B.Cu") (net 2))
 (segment (start 166.620001 78.020001) (end 157.04 78.020001) (width 0.25) (layer "B.Cu") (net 2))
 (segment (start 151.73 100.95) (end 145.87 95.09) (width 0.25) (layer "B.Cu") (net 2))
 (segment (start 151.51 100.82) (end 148.75 98.06) (width 0.25) (layer "B.Cu") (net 2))
 (segment (start 167.5125 98.025) (end 148.785 98.025) (width 0.25) (layer "B.Cu") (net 2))
 (segment (start 149.46 100.95) (end 149.46 104.81) (width 0.25) (layer "F.Cu") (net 9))
 (segment (start 149.46 104.81) (end 151.05 106.4) (width 0.25) (layer "F.Cu") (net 9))
 (segment (start 157.24 105.09) (end 155.93 106.4) (width 0.25) (layer "F.Cu") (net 8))
 (segment (start 157.24 100.82) (end 157.24 105.09) (width 0.25) (layer "F.Cu") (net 8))
 (segment (start 139.795 105.84) (end 139.795 101.005) (width 0.25) (layer "F.Cu") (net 30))
 (segment (start 139.795 101.005) (end 138.65 99.86) (width 0.25) (layer "F.Cu") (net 30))
 (segment (start 156.55 95.58) (end 160.36 99.39) (width 0.25) (layer "F.Cu") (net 4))
 (segment (start 167.999201 99.39) (end 168.86 100.250799) (width 0.25) (layer "F.Cu") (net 4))
 (segment (start 168.86 101.9125) (end 170.0525 103.105) (width 0.25) (layer "F.Cu") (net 4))
 (segment (start 160.36 99.39) (end 167.999201 99.39) (width 0.25) (layer "F.Cu") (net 4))
 (segment (start 168.86 100.250799) (end 168.86 101.9125) (width 0.25) (layer "F.Cu") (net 4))
 (segment (start 155.35 91.73) (end 154.68 91.06) (width 0.25) (layer "F.Cu") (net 3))
 (segment (start 158 93.33) (end 156.95 93.33) (width 0.25) (layer "F.Cu") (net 3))
 (segment (start 159.135 78.235) (end 163.830965 78.235) (width 0.25) (layer "F.Cu") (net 3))
 (segment (start 159.05 91.73) (end 158 91.73) (width 0.25) (layer "F.Cu") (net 3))
 (segment (start 158 91.73) (end 155.35 91.73) (width 0.25) (layer "F.Cu") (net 3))
 (segment (start 160.42 90.36) (end 159.05 91.73) (width 0.25) (layer "F.Cu") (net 3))
 (segment (start 154.68 91.06) (end 154.55 90.93) (width 0.25) (layer "F.Cu") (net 3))
 (segment (start 154.55 90.93) (end 149.5 90.93) (width 0.25) (layer "F.Cu") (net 3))
 (segment (start 164.74 80.44) (end 160.42 84.76) (width 0.25) (layer "F.Cu") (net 3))
 (segment (start 160.42 84.76) (end 160.42 90.36) (width 0.25) (layer "F.Cu") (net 3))
 (segment (start 168.6875 104.28) (end 170.96 104.28) (width 0.25) (layer "F.Cu") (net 3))
 (segment (start 163.830965 78.235) (end 164.74 79.144035) (width 0.25) (layer "F.Cu") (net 3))
 (segment (start 167.019201 93.33) (end 158 93.33) (width 0.25) (layer "F.Cu") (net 3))
 (segment (start 171.23 97.540799) (end 167.019201 93.33) (width 0.25) (layer "F.Cu") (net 3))
 (segment (start 171.23 104.01) (end 171.23 97.540799) (width 0.25) (layer "F.Cu") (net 3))
 (segment (start 164.74 79.144035) (end 164.74 80.44) (width 0.25) (layer "F.Cu") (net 3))
 (segment (start 167.5125 103.105) (end 168.6875 104.28) (width 0.25) (layer "F.Cu") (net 3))
 (segment (start 170.96 104.28) (end 171.23 104.01) (width 0.25) (layer "F.Cu") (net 3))
 (segment (start 156.95 93.33) (end 154.68 91.06) (width 0.25) (layer "F.Cu") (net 3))
 (segment (start 155.54 81.83) (end 159.135 78.235) (width 0.25) (layer "F.Cu") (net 3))
 (segment (start 170.0525 100.565) (end 168.6875 99.2) (width 0.25) (layer "F.Cu") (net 5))
 (segment (start 168.6875 97.538299) (end 165.279201 94.13) (width 0.25) (layer "F.Cu") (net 5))
 (segment (start 165.279201 94.13) (end 158 94.13) (width 0.25) (layer "F.Cu") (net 5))
 (segment (start 168.6875 99.2) (end 168.6875 97.538299) (width 0.25) (layer "F.Cu") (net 5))
 (segment (start 155.75 96.63) (end 159.685 100.565) (width 0.25) (layer "F.Cu") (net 6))
 (segment (start 159.685 100.565) (end 167.5125 100.565) (width 0.25) (layer "F.Cu") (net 6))
 (segment (start 155.75 95.58) (end 155.75 96.63) (width 0.25) (layer "F.Cu") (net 6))
 (segment (start 160.42 79.68) (end 161.415 78.685) (width 0.25) (layer "F.Cu") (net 7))
 (segment (start 160.759569 83.62) (end 157.99 83.62) (width 0.25) (layer "F.Cu") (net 7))
 (segment (start 157.91 85.58) (end 157.91 83.7) (width 0.25) (layer "F.Cu") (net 7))
 (segment (start 166.94 92.33) (end 166.94 91.91) (width 0.25) (layer "F.Cu") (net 7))
 (segment (start 164.245 80.134569) (end 160.759569 83.62) (width 0.25) (layer "F.Cu") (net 7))
 (segment (start 161.415 78.685) (end 163.644569 78.685) (width 0.25) (layer "F.Cu") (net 7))
 (segment (start 154.545 83.62) (end 153.35 84.815) (width 0.25) (layer "F.Cu") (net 7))
 (segment (start 164.245 79.285431) (end 164.245 80.134569) (width 0.25) (layer "F.Cu") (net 7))
 (segment (start 166.94 91.91) (end 161.99 86.96) (width 0.25) (layer "F.Cu") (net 7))
 (segment (start 170.0525 98.025) (end 166.9119 94.8844) (width 0.25) (layer "F.Cu") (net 7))
 (segment (start 153.35 84.815) (end 153.35 87.08) (width 0.25) (layer "F.Cu") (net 7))
 (segment (start 163.644569 78.685) (end 164.245 79.285431) (width 0.25) (layer "F.Cu") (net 7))
 (segment (start 166.9119 94.8844) (end 166.9119 94.7381) (width 0.25) (layer "F.Cu") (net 7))
 (segment (start 157.99 83.62) (end 154.545 83.62) (width 0.25) (layer "F.Cu") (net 7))
 (segment (start 157.91 83.7) (end 157.99 83.62) (width 0.25) (layer "F.Cu") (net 7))
 (via (at 161.99 86.96) (size 0.8) (drill 0.4) (layers "F.Cu" "B.Cu") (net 7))
 (via (at 157.91 85.58) (size 0.8) (drill 0.4) (layers "F.Cu" "B.Cu") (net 7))
 (via (at 166.94 92.33) (size 0.8) (drill 0.4) (layers "F.Cu" "B.Cu") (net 7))
 (via (at 166.9119 94.7381) (size 0.8) (drill 0.4) (layers "F.Cu" "B.Cu") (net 7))
 (segment (start 161.99 86.96) (end 159.41 86.96) (width 0.25) (layer "B.Cu") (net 7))
 (segment (start 166.9119 94.7381) (end 166.9119 92.3581) (width 0.25) (layer "B.Cu") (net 7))
 (segment (start 166.9119 92.3581) (end 166.94 92.33) (width 0.25) (layer "B.Cu") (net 7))
 (segment (start 159.41 86.96) (end 158.03 85.58) (width 0.25) (layer "B.Cu") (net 7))
 (segment (start 158.03 85.58) (end 157.91 85.58) (width 0.25) (layer "B.Cu") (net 7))
 (segment (start 163.22 79.71) (end 159.775 83.155) (width 0.25) (layer "F.Cu") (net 1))
 (segment (start 159.775 83.155) (end 151.785 83.155) (width 0.25) (layer "F.Cu") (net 1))
 (segment (start 150.46 81.83) (end 148.87 81.83) (width 0.25) (layer "F.Cu") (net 1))
 (segment (start 148.87 81.83) (end 140.79 89.91) (width 0.25) (layer "F.Cu") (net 1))
 (segment (start 151.785 83.155) (end 150.46 81.83) (width 0.25) (layer "F.Cu") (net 1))
 (segment (start 164.87 86.44) (end 163.22 84.79) (width 0.25) (layer "F.Cu") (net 10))
 (segment (start 167.42 86.44) (end 164.87 86.44) (width 0.25) (layer "F.Cu") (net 10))
 (segment (start 147.66 89.445) (end 148.575 88.53) (width 0.25) (layer "F.Cu") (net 12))
 (segment (start 147.66 95.93) (end 147.66 89.445) (width 0.25) (layer "F.Cu") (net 12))
 (segment (start 148.575 88.53) (end 149.5 88.53) (width 0.25) (layer "F.Cu") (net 12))
 (segment (start 143.73 99.86) (end 147.66 95.93) (width 0.25) (layer "F.Cu") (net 12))
 (segment (start 169.96 86.44) (end 171.68 88.16) (width 0.25) (layer "F.Cu") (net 11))
 (segment (start 148.575 89.33) (end 149.5 89.33) (width 0.25) (layer "F.Cu") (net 11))
 (segment (start 171.68 88.16) (end 171.68 104.196396) (width 0.25) (layer "F.Cu") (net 11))
 (segment (start 154.78 96.73) (end 150.375 96.73) (width 0.25) (layer "F.Cu") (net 11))
 (segment (start 148.375 89.53) (end 148.575 89.33) (width 0.25) (layer "F.Cu") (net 11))
 (segment (start 171.146396 104.73) (end 162.78 104.73) (width 0.25) (layer "F.Cu") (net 11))
 (segment (start 148.375 94.73) (end 148.375 89.53) (width 0.25) (layer "F.Cu") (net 11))
 (segment (start 171.68 104.196396) (end 171.146396 104.73) (width 0.25) (layer "F.Cu") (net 11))
 (segment (start 150.375 96.73) (end 148.375 94.73) (width 0.25) (layer "F.Cu") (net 11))
 (segment (start 162.78 104.73) (end 154.78 96.73) (width 0.25) (layer "F.Cu") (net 11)))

